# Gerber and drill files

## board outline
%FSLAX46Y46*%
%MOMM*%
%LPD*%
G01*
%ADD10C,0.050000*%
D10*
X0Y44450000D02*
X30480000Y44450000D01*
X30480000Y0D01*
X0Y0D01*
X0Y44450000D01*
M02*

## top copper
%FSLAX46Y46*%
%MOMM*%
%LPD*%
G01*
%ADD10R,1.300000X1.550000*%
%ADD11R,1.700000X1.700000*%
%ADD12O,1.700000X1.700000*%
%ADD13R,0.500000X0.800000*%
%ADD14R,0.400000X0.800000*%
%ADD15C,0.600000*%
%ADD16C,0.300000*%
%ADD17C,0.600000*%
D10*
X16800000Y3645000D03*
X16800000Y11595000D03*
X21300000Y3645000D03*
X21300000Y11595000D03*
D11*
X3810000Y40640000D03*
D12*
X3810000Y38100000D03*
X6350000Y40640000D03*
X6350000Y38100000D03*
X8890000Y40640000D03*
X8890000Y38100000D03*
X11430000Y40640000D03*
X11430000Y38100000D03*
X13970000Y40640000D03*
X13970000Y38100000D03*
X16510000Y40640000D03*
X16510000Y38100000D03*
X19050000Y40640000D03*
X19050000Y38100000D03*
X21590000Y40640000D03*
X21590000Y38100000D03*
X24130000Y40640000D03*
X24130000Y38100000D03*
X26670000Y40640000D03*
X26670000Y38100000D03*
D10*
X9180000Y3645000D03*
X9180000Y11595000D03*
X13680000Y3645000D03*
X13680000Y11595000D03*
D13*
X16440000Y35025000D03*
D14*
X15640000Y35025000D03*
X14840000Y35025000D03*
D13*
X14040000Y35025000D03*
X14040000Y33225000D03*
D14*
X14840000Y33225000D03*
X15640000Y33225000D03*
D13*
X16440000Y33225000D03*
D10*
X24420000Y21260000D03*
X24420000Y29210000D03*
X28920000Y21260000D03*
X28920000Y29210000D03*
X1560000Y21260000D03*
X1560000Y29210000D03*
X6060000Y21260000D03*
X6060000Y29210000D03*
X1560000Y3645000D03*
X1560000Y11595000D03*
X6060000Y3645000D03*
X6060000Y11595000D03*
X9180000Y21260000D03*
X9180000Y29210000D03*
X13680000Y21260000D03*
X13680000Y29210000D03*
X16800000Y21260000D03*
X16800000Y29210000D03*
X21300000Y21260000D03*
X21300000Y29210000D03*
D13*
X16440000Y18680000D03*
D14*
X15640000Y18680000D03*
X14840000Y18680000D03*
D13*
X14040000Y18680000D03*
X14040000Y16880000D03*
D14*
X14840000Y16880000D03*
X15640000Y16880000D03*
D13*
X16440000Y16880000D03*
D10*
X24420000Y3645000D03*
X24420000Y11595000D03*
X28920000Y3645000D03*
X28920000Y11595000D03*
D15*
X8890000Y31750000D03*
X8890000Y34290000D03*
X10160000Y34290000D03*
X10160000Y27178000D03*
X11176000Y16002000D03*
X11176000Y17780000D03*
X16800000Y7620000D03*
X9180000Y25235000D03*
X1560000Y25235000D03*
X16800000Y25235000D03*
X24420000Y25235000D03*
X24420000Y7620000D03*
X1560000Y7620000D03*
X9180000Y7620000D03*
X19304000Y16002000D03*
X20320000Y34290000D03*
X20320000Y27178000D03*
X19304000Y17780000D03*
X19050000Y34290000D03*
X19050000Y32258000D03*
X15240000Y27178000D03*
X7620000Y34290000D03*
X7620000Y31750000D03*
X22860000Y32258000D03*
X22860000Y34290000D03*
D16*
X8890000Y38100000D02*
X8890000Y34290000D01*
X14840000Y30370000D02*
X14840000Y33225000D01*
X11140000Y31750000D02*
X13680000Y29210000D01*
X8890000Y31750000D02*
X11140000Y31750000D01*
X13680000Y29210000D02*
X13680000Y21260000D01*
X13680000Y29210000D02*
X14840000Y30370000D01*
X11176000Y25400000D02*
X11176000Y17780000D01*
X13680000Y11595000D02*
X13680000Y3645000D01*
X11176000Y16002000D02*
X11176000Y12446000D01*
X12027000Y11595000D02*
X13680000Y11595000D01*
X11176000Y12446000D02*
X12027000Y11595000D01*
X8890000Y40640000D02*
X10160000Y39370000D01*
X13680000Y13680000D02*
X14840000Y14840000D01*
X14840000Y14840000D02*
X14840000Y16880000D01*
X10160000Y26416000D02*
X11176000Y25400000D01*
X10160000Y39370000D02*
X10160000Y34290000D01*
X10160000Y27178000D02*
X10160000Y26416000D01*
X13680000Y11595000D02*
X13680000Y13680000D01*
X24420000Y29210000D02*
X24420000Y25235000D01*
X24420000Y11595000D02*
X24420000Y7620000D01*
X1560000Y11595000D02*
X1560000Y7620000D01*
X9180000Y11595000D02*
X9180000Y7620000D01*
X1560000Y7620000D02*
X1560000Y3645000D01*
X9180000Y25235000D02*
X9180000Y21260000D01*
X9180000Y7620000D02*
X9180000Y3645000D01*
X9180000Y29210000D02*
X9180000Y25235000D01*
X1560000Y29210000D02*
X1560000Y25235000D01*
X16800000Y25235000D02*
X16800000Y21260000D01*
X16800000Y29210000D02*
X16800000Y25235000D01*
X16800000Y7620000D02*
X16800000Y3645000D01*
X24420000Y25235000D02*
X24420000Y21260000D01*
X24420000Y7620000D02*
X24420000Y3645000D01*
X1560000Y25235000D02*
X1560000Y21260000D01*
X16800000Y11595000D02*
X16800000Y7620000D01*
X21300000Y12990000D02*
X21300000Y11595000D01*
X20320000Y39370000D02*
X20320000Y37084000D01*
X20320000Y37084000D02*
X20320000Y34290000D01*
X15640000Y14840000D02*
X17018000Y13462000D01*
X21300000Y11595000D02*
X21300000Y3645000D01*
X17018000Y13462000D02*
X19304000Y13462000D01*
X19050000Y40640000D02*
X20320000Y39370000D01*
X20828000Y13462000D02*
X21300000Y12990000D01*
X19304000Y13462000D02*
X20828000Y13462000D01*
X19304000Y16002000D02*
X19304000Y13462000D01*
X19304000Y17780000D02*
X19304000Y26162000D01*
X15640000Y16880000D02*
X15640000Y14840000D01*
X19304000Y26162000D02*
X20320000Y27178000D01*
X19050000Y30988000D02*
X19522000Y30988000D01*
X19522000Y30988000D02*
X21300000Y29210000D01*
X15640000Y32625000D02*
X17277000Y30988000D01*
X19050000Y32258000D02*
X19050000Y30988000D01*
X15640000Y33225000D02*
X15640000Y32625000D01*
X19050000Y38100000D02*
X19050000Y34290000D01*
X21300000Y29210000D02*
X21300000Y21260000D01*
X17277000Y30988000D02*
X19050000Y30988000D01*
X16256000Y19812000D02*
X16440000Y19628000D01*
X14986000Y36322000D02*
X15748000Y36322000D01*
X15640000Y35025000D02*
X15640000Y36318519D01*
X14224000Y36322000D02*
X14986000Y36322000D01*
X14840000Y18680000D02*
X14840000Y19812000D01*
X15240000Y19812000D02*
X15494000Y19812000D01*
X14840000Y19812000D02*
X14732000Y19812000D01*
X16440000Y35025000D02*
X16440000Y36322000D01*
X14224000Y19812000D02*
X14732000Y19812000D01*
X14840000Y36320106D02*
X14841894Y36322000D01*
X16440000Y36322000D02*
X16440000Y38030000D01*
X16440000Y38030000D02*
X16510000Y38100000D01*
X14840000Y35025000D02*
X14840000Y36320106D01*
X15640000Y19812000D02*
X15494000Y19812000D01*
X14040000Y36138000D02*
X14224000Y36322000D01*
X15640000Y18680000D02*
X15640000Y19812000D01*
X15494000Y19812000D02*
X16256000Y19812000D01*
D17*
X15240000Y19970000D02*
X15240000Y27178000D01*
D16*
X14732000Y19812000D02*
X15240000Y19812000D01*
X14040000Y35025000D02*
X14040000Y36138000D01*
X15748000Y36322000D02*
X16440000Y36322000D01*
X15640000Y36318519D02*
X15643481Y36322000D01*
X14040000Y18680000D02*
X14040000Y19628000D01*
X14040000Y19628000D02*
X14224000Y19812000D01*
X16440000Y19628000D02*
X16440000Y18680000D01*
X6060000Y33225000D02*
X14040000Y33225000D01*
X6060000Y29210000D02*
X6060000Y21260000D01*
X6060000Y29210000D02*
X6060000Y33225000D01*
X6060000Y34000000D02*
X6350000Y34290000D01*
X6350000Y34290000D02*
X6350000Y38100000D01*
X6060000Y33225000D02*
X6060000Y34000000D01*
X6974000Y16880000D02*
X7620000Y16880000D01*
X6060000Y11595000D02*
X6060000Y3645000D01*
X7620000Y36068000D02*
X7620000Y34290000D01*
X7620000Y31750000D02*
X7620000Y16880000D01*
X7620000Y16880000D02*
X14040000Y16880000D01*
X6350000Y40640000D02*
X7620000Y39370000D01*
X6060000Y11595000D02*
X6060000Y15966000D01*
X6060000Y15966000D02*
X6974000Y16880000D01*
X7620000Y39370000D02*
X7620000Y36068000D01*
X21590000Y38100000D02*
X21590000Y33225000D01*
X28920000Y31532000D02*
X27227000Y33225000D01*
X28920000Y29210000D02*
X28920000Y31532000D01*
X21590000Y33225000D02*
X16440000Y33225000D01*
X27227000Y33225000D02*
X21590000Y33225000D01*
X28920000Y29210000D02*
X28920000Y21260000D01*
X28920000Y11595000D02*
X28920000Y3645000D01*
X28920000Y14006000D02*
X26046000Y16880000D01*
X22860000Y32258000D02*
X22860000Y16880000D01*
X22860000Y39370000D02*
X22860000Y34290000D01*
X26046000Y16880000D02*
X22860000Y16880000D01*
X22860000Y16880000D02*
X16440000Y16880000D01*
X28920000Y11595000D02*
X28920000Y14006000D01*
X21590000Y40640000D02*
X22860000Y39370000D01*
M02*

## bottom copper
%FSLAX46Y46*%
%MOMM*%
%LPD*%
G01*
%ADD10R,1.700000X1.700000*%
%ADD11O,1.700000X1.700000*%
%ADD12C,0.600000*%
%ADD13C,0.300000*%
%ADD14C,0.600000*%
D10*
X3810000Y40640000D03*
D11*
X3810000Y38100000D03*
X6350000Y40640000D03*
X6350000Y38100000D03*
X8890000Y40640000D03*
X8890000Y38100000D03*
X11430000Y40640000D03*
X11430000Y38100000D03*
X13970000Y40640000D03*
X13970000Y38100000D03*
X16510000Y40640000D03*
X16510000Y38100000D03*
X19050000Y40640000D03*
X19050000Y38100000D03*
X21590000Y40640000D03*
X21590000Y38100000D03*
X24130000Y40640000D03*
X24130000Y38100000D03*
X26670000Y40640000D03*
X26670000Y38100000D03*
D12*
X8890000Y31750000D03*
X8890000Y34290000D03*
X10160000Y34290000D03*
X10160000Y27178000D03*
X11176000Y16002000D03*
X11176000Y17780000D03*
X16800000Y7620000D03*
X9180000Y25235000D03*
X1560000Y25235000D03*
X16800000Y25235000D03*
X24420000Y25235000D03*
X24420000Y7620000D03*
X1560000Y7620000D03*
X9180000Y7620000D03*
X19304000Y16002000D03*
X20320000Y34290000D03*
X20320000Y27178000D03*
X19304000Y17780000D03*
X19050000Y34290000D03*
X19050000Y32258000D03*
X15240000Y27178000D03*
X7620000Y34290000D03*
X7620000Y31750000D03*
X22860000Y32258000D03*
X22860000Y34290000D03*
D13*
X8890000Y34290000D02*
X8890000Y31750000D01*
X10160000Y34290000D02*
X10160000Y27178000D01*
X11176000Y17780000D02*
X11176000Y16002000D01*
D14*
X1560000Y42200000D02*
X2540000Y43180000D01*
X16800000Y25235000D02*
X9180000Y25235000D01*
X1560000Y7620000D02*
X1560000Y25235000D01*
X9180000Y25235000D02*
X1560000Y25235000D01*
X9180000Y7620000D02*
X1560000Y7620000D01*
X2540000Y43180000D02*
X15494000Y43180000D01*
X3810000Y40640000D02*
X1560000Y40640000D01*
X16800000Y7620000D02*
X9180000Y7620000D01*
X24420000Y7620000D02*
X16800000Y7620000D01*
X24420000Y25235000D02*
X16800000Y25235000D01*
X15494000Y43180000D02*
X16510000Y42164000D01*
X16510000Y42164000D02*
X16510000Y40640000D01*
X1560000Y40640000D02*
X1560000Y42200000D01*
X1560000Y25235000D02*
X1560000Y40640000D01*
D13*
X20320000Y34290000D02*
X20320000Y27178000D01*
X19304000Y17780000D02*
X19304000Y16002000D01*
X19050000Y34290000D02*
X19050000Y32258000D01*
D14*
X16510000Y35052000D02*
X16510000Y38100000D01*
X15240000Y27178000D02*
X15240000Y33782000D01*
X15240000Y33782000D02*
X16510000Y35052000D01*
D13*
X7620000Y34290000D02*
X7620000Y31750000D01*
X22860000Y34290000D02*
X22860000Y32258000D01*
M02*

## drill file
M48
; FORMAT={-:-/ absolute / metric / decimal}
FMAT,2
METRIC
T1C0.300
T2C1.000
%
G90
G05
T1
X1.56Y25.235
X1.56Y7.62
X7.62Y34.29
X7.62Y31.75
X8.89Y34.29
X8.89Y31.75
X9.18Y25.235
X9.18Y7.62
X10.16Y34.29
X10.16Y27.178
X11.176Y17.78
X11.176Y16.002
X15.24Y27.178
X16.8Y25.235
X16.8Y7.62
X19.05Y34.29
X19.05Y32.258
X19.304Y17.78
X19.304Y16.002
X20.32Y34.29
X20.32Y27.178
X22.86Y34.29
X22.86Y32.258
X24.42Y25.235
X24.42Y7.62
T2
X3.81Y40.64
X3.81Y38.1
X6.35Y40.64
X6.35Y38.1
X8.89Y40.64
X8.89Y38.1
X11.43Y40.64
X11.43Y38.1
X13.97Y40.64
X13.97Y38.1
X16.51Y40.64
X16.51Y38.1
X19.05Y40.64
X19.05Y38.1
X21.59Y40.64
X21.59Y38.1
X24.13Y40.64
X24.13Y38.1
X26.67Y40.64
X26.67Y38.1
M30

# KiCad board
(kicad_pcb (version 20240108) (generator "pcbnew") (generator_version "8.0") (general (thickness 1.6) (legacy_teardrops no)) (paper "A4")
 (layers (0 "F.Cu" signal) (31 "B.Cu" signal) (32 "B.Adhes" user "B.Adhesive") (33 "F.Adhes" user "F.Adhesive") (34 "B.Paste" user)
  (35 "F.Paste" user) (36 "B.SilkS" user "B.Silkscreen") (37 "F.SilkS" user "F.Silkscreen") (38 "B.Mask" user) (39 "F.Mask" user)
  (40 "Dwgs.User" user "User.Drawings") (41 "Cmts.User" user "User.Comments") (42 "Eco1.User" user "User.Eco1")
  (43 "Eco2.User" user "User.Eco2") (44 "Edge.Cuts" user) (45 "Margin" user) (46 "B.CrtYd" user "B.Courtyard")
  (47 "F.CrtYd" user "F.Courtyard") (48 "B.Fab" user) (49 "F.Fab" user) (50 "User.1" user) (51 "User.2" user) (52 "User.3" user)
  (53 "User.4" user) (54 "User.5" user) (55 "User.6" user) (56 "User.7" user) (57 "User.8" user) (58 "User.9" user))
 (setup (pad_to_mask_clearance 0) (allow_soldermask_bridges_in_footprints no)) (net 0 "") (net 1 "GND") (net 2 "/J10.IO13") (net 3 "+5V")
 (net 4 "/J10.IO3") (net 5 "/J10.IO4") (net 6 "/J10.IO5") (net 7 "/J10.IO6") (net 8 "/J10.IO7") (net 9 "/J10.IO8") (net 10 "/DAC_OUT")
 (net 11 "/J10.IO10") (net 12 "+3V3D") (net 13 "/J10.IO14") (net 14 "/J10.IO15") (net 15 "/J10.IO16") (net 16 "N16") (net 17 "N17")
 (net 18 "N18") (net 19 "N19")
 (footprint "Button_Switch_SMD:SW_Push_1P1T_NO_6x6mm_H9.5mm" (layer "F.Cu") (at 19.05 -7.62 90)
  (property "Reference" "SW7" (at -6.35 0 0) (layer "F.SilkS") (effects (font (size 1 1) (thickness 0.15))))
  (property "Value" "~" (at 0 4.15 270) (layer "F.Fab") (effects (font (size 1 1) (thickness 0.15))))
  (pad "1" smd rect (at -3.975 -2.25 90) (size 1.55 1.3) (layers "F.Cu" "F.Paste" "F.Mask") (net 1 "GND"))
  (pad "1" smd rect (at 3.975 -2.25 90) (size 1.55 1.3) (layers "F.Cu" "F.Paste" "F.Mask") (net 1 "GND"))
  (pad "2" smd rect (at -3.975 2.25 90) (size 1.55 1.3) (layers "F.Cu" "F.Paste" "F.Mask") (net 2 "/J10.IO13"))
  (pad "2" smd rect (at 3.975 2.25 90) (size 1.55 1.3) (layers "F.Cu" "F.Paste" "F.Mask") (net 2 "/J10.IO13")))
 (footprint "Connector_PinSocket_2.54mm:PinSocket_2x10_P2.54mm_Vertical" (layer "F.Cu") (at 3.81 -40.64 90)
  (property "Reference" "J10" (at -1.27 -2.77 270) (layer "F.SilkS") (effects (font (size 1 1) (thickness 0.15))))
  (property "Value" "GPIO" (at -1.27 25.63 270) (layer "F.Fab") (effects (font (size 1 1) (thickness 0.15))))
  (pad "1" thru_hole rect (at 0 0 90) (size 1.7 1.7) (drill 1) (layers "*.Cu" "*.Mask") (remove_unused_layers no) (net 1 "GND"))
  (pad "2" thru_hole oval (at -2.54 0 90) (size 1.7 1.7) (drill 1) (layers "*.Cu" "*.Mask") (remove_unused_layers no) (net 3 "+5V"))
  (pad "3" thru_hole oval (at 0 2.54 90) (size 1.7 1.7) (drill 1) (layers "*.Cu" "*.Mask") (remove_unused_layers no) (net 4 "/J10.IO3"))
  (pad "4" thru_hole oval (at -2.54 2.54 90) (size 1.7 1.7) (drill 1) (layers "*.Cu" "*.Mask") (remove_unused_layers no) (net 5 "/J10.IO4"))
  (pad "5" thru_hole oval (at 0 5.08 90) (size 1.7 1.7) (drill 1) (layers "*.Cu" "*.Mask") (remove_unused_layers no) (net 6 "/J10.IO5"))
  (pad "6" thru_hole oval (at -2.54 5.08 90) (size 1.7 1.7) (drill 1) (layers "*.Cu" "*.Mask") (remove_unused_layers no) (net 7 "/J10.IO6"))
  (pad "7" thru_hole oval (at 0 7.62 90) (size 1.7 1.7) (drill 1) (layers "*.Cu" "*.Mask") (remove_unused_layers no) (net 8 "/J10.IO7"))
  (pad "8" thru_hole oval (at -2.54 7.62 90) (size 1.7 1.7) (drill 1) (layers "*.Cu" "*.Mask") (remove_unused_layers no) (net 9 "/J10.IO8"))
  (pad "9" thru_hole oval (at 0 10.16 90) (size 1.7 1.7) (drill 1) (layers "*.Cu" "*.Mask") (remove_unused_layers no) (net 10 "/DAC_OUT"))
  (pad "10" thru_hole oval (at -2.54 10.16 90) (size 1.7 1.7) (drill 1) (layers "*.Cu" "*.Mask") (remove_unused_layers no)
   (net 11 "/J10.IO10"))
  (pad "11" thru_hole oval (at 0 12.7 90) (size 1.7 1.7) (drill 1) (layers "*.Cu" "*.Mask") (remove_unused_layers no) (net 1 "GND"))
  (pad "12" thru_hole oval (at -2.54 12.7 90) (size 1.7 1.7) (drill 1) (layers "*.Cu" "*.Mask") (remove_unused_layers no) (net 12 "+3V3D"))
  (pad "13" thru_hole oval (at 0 15.24 90) (size 1.7 1.7) (drill 1) (layers "*.Cu" "*.Mask") (remove_unused_layers no) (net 2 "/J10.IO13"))
  (pad "14" thru_hole oval (at -2.54 15.24 90) (size 1.7 1.7) (drill 1) (layers "*.Cu" "*.Mask") (remove_unused_layers no)
   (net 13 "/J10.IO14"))
  (pad "15" thru_hole oval (at 0 17.78 90) (size 1.7 1.7) (drill 1) (layers "*.Cu" "*.Mask") (remove_unused_layers no) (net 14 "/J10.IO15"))
  (pad "16" thru_hole oval (at -2.54 17.78 90) (size 1.7 1.7) (drill 1) (layers "*.Cu" "*.Mask") (remove_unused_layers no)
   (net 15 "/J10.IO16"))
  (pad "17" thru_hole oval (at 0 20.32 90) (size 1.7 1.7) (drill 1) (layers "*.Cu" "*.Mask") (remove_unused_layers no) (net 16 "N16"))
  (pad "18" thru_hole oval (at -2.54 20.32 90) (size 1.7 1.7) (drill 1) (layers "*.Cu" "*.Mask") (remove_unused_layers no) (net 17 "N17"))
  (pad "19" thru_hole oval (at 0 22.86 90) (size 1.7 1.7) (drill 1) (layers "*.Cu" "*.Mask") (remove_unused_layers no) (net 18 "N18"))
  (pad "20" thru_hole oval (at -2.54 22.86 90) (size 1.7 1.7) (drill 1) (layers "*.Cu" "*.Mask") (remove_unused_layers no) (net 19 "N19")))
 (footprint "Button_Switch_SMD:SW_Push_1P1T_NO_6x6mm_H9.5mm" (layer "F.Cu") (at 11.43 -7.62 90)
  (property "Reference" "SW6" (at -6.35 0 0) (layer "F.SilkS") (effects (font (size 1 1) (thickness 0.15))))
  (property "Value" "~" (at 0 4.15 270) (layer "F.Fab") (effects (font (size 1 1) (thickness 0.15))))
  (pad "1" smd rect (at -3.975 -2.25 90) (size 1.55 1.3) (layers "F.Cu" "F.Paste" "F.Mask") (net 1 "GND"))
  (pad "1" smd rect (at 3.975 -2.25 90) (size 1.55 1.3) (layers "F.Cu" "F.Paste" "F.Mask") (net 1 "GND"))
  (pad "2" smd rect (at -3.975 2.25 90) (size 1.55 1.3) (layers "F.Cu" "F.Paste" "F.Mask") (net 6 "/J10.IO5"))
  (pad "2" smd rect (at 3.975 2.25 90) (size 1.55 1.3) (layers "F.Cu" "F.Paste" "F.Mask") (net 6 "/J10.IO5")))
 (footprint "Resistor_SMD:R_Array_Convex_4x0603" (layer "F.Cu") (at 15.24 -34.125 -90)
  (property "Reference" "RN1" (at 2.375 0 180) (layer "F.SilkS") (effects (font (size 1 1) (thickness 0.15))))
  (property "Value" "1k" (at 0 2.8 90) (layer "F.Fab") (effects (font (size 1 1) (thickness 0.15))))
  (pad "1" smd rect (at -0.9 -1.2 270) (size 0.8 0.5) (layers "F.Cu" "F.Paste" "F.Mask") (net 12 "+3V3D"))
  (pad "2" smd rect (at -0.9 -0.4 270) (size 0.8 0.4) (layers "F.Cu" "F.Paste" "F.Mask") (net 12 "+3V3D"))
  (pad "3" smd rect (at -0.9 0.4 270) (size 0.8 0.4) (layers "F.Cu" "F.Paste" "F.Mask") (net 12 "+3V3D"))
  (pad "4" smd rect (at -0.9 1.2 270) (size 0.8 0.5) (layers "F.Cu" "F.Paste" "F.Mask") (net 12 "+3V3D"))
  (pad "5" smd rect (at 0.9 1.2 270) (size 0.8 0.5) (layers "F.Cu" "F.Paste" "F.Mask") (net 5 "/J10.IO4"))
  (pad "6" smd rect (at 0.9 0.4 270) (size 0.8 0.4) (layers "F.Cu" "F.Paste" "F.Mask") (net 7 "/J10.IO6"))
  (pad "7" smd rect (at 0.9 -0.4 270) (size 0.8 0.4) (layers "F.Cu" "F.Paste" "F.Mask") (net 13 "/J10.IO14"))
  (pad "8" smd rect (at 0.9 -1.2 270) (size 0.8 0.5) (layers "F.Cu" "F.Paste" "F.Mask") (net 15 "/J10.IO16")))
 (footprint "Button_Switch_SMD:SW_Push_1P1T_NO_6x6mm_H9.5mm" (layer "F.Cu") (at 26.67 -25.235 90)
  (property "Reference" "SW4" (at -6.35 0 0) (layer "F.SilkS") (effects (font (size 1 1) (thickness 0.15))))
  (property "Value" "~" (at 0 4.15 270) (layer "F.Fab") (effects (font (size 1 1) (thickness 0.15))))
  (pad "1" smd rect (at -3.975 -2.25 90) (size 1.55 1.3) (layers "F.Cu" "F.Paste" "F.Mask") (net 1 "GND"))
  (pad "1" smd rect (at 3.975 -2.25 90) (size 1.55 1.3) (layers "F.Cu" "F.Paste" "F.Mask") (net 1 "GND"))
  (pad "2" smd rect (at -3.975 2.25 90) (size 1.55 1.3) (layers "F.Cu" "F.Paste" "F.Mask") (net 15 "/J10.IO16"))
  (pad "2" smd rect (at 3.975 2.25 90) (size 1.55 1.3) (layers "F.Cu" "F.Paste" "F.Mask") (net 15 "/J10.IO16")))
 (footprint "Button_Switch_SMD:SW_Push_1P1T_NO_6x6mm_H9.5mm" (layer "F.Cu") (at 3.81 -25.235 90)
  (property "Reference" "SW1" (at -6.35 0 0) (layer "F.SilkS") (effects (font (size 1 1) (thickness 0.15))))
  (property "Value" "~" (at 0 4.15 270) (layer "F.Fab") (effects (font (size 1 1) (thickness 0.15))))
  (pad "1" smd rect (at -3.975 -2.25 90) (size 1.55 1.3) (layers "F.Cu" "F.Paste" "F.Mask") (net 1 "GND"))
  (pad "1" smd rect (at 3.975 -2.25 90) (size 1.55 1.3) (layers "F.Cu" "F.Paste" "F.Mask") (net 1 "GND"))
  (pad "2" smd rect (at -3.975 2.25 90) (size 1.55 1.3) (layers "F.Cu" "F.Paste" "F.Mask") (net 5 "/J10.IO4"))
  (pad "2" smd rect (at 3.975 2.25 90) (size 1.55 1.3) (layers "F.Cu" "F.Paste" "F.Mask") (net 5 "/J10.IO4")))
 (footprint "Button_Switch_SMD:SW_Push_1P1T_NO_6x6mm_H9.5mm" (layer "F.Cu") (at 3.81 -7.62 90)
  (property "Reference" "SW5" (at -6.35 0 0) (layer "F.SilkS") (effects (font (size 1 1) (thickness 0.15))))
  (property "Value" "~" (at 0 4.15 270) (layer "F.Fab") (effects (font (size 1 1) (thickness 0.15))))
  (pad "1" smd rect (at -3.975 -2.25 90) (size 1.55 1.3) (layers "F.Cu" "F.Paste" "F.Mask") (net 1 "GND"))
  (pad "1" smd rect (at 3.975 -2.25 90) (size 1.55 1.3) (layers "F.Cu" "F.Paste" "F.Mask") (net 1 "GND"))
  (pad "2" smd rect (at -3.975 2.25 90) (size 1.55 1.3) (layers "F.Cu" "F.Paste" "F.Mask") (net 4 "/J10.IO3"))
  (pad "2" smd rect (at 3.975 2.25 90) (size 1.55 1.3) (layers "F.Cu" "F.Paste" "F.Mask") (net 4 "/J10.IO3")))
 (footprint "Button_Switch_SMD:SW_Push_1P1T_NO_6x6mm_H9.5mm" (layer "F.Cu") (at 11.43 -25.235 90)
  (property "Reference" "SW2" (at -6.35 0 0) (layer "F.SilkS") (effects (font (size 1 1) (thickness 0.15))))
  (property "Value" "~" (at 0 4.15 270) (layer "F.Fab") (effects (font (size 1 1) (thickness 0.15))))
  (pad "1" smd rect (at -3.975 -2.25 90) (size 1.55 1.3) (layers "F.Cu" "F.Paste" "F.Mask") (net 1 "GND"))
  (pad "1" smd rect (at 3.975 -2.25 90) (size 1.55 1.3) (layers "F.Cu" "F.Paste" "F.Mask") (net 1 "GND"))
  (pad "2" smd rect (at -3.975 2.25 90) (size 1.55 1.3) (layers "F.Cu" "F.Paste" "F.Mask") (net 7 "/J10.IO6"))
  (pad "2" smd rect (at 3.975 2.25 90) (size 1.55 1.3) (layers "F.Cu" "F.Paste" "F.Mask") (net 7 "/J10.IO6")))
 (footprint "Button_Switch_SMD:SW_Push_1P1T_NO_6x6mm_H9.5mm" (layer "F.Cu") (at 19.05 -25.235 90)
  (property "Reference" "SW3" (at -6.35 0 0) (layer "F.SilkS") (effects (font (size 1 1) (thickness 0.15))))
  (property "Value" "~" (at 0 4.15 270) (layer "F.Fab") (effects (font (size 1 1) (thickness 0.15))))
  (pad "1" smd rect (at -3.975 -2.25 90) (size 1.55 1.3) (layers "F.Cu" "F.Paste" "F.Mask") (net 1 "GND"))
  (pad "1" smd rect (at 3.975 -2.25 90) (size 1.55 1.3) (layers "F.Cu" "F.Paste" "F.Mask") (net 1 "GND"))
  (pad "2" smd rect (at -3.975 2.25 90) (size 1.55 1.3) (layers "F.Cu" "F.Paste" "F.Mask") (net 13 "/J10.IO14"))
  (pad "2" smd rect (at 3.975 2.25 90) (size 1.55 1.3) (layers "F.Cu" "F.Paste" "F.Mask") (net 13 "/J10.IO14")))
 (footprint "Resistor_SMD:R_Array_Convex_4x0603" (layer "F.Cu") (at 15.24 -17.78 -90)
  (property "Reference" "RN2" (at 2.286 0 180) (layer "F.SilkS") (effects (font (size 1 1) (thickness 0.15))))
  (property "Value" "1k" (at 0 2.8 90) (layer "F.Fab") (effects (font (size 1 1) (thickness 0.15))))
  (pad "1" smd rect (at -0.9 -1.2 270) (size 0.8 0.5) (layers "F.Cu" "F.Paste" "F.Mask") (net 12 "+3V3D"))
  (pad "2" smd rect (at -0.9 -0.4 270) (size 0.8 0.4) (layers "F.Cu" "F.Paste" "F.Mask") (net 12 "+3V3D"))
  (pad "3" smd rect (at -0.9 0.4 270) (size 0.8 0.4) (layers "F.Cu" "F.Paste" "F.Mask") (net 12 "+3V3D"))
  (pad "4" smd rect (at -0.9 1.2 270) (size 0.8 0.5) (layers "F.Cu" "F.Paste" "F.Mask") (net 12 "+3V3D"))
  (pad "5" smd rect (at 0.9 1.2 270) (size 0.8 0.5) (layers "F.Cu" "F.Paste" "F.Mask") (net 4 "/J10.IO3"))
  (pad "6" smd rect (at 0.9 0.4 270) (size 0.8 0.4) (layers "F.Cu" "F.Paste" "F.Mask") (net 6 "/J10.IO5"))
  (pad "7" smd rect (at 0.9 -0.4 270) (size 0.8 0.4) (layers "F.Cu" "F.Paste" "F.Mask") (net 2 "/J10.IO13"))
  (pad "8" smd rect (at 0.9 -1.2 270) (size 0.8 0.5) (layers "F.Cu" "F.Paste" "F.Mask") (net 14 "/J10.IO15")))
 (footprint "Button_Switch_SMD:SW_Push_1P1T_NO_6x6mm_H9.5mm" (layer "F.Cu") (at 26.67 -7.62 90)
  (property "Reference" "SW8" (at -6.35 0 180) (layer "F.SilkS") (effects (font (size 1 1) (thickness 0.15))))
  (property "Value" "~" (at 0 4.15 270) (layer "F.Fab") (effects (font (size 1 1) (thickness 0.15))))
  (pad "1" smd rect (at -3.975 -2.25 90) (size 1.55 1.3) (layers "F.Cu" "F.Paste" "F.Mask") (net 1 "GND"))
  (pad "1" smd rect (at 3.975 -2.25 90) (size 1.55 1.3) (layers "F.Cu" "F.Paste" "F.Mask") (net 1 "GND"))
  (pad "2" smd rect (at -3.975 2.25 90) (size 1.55 1.3) (layers "F.Cu" "F.Paste" "F.Mask") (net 14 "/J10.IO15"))
  (pad "2" smd rect (at 3.975 2.25 90) (size 1.55 1.3) (layers "F.Cu" "F.Paste" "F.Mask") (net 14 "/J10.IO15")))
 (gr_rect (start 0 -44.45) (end 30.48 0) (stroke (width 0.05) (type default)) (fill none) (layer "Edge.Cuts"))
 (segment (start 8.89 -38.1) (end 8.89 -34.29) (width 0.3) (layer "F.Cu") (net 7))
 (segment (start 14.84 -30.37) (end 14.84 -33.225) (width 0.3) (layer "F.Cu") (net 7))
 (segment (start 11.14 -31.75) (end 13.68 -29.21) (width 0.3) (layer "F.Cu") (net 7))
 (segment (start 8.89 -31.75) (end 11.14 -31.75) (width 0.3) (layer "F.Cu") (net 7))
 (segment (start 13.68 -29.21) (end 13.68 -21.26) (width 0.3) (layer "F.Cu") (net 7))
 (segment (start 13.68 -29.21) (end 14.84 -30.37) (width 0.3) (layer "F.Cu") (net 7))
 (via (at 8.89 -31.75) (size 0.6) (drill 0.3) (layers "F.Cu" "B.Cu") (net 7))
 (via (at 8.89 -34.29) (size 0.6) (drill 0.3) (layers "F.Cu" "B.Cu") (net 7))
 (segment (start 8.89 -34.29) (end 8.89 -31.75) (width 0.3) (layer "B.Cu") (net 7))
 (segment (start 11.176 -25.4) (end 11.176 -17.78) (width 0.3) (layer "F.Cu") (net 6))
 (segment (start 13.68 -11.595) (end 13.68 -3.645) (width 0.3) (layer "F.Cu") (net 6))
 (segment (start 11.176 -16.002) (end 11.176 -12.446) (width 0.3) (layer "F.Cu") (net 6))
 (segment (start 12.027 -11.595) (end 13.68 -11.595) (width 0.3) (layer "F.Cu") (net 6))
 (segment (start 11.176 -12.446) (end 12.027 -11.595) (width 0.3) (layer "F.Cu") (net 6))
 (segment (start 8.89 -40.64) (end 10.16 -39.37) (width 0.3) (layer "F.Cu") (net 6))
 (segment (start 13.68 -13.68) (end 14.84 -14.84) (width 0.3) (layer "F.Cu") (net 6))
 (segment (start 14.84 -14.84) (end 14.84 -16.88) (width 0.3) (layer "F.Cu") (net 6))
 (segment (start 10.16 -26.416) (end 11.176 -25.4) (width 0.3) (layer "F.Cu") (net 6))
 (segment (start 10.16 -39.37) (end 10.16 -34.29) (width 0.3) (layer "F.Cu") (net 6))
 (segment (start 10.16 -27.178) (end 10.16 -26.416) (width 0.3) (layer "F.Cu") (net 6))
 (segment (start 13.68 -11.595) (end 13.68 -13.68) (width 0.3) (layer "F.Cu") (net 6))
 (via (at 10.16 -34.29) (size 0.6) (drill 0.3) (layers "F.Cu" "B.Cu") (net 6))
 (via (at 10.16 -27.178) (size 0.6) (drill 0.3) (layers "F.Cu" "B.Cu") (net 6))
 (via (at 11.176 -16.002) (size 0.6) (drill 0.3) (layers "F.Cu" "B.Cu") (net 6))
 (via (at 11.176 -17.78) (size 0.6) (drill 0.3) (layers "F.Cu" "B.Cu") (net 6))
 (segment (start 10.16 -34.29) (end 10.16 -27.178) (width 0.3) (layer "B.Cu") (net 6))
 (segment (start 11.176 -17.78) (end 11.176 -16.002) (width 0.3) (layer "B.Cu") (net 6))
 (segment (start 24.42 -29.21) (end 24.42 -25.235) (width 0.3) (layer "F.Cu") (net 1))
 (segment (start 24.42 -11.595) (end 24.42 -7.62) (width 0.3) (layer "F.Cu") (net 1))
 (segment (start 1.56 -11.595) (end 1.56 -7.62) (width 0.3) (layer "F.Cu") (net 1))
 (segment (start 9.18 -11.595) (end 9.18 -7.62) (width 0.3) (layer "F.Cu") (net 1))
 (segment (start 1.56 -7.62) (end 1.56 -3.645) (width 0.3) (layer "F.Cu") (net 1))
 (segment (start 9.18 -25.235) (end 9.18 -21.26) (width 0.3) (layer "F.Cu") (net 1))
 (segment (start 9.18 -7.62) (end 9.18 -3.645) (width 0.3) (layer "F.Cu") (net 1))
 (segment (start 9.18 -29.21) (end 9.18 -25.235) (width 0.3) (layer "F.Cu") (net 1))
 (segment (start 1.56 -29.21) (end 1.56 -25.235) (width 0.3) (layer "F.Cu") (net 1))
 (segment (start 16.8 -25.235) (end 16.8 -21.26) (width 0.3) (layer "F.Cu") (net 1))
 (segment (start 16.8 -29.21) (end 16.8 -25.235) (width 0.3) (layer "F.Cu") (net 1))
 (segment (start 16.8 -7.62) (end 16.8 -3.645) (width 0.3) (layer "F.Cu") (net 1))
 (segment (start 24.42 -25.235) (end 24.42 -21.26) (width 0.3) (layer "F.Cu") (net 1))
 (segment (start 24.42 -7.62) (end 24.42 -3.645) (width 0.3) (layer "F.Cu") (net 1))
 (segment (start 1.56 -25.235) (end 1.56 -21.26) (width 0.3) (layer "F.Cu") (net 1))
 (segment (start 16.8 -11.595) (end 16.8 -7.62) (width 0.3) (layer "F.Cu") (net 1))
 (via (at 16.8 -7.62) (size 0.6) (drill 0.3) (layers "F.Cu" "B.Cu") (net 1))
 (via (at 9.18 -25.235) (size 0.6) (drill 0.3) (layers "F.Cu" "B.Cu") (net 1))
 (via (at 1.56 -25.235) (size 0.6) (drill 0.3) (layers "F.Cu" "B.Cu") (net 1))
 (via (at 16.8 -25.235) (size 0.6) (drill 0.3) (layers "F.Cu" "B.Cu") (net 1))
 (via (at 24.42 -25.235) (size 0.6) (drill 0.3) (layers "F.Cu" "B.Cu") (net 1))
 (via (at 24.42 -7.62) (size 0.6) (drill 0.3) (layers "F.Cu" "B.Cu") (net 1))
 (via (at 1.56 -7.62) (size 0.6) (drill 0.3) (layers "F.Cu" "B.Cu") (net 1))
 (via (at 9.18 -7.62) (size 0.6) (drill 0.3) (layers "F.Cu" "B.Cu") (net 1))
 (segment (start 1.56 -42.2) (end 2.54 -43.18) (width 0.6) (layer "B.Cu") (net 1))
 (segment (start 16.8 -25.235) (end 9.18 -25.235) (width 0.6) (layer "B.Cu") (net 1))
 (segment (start 1.56 -7.62) (end 1.56 -25.235) (width 0.6) (layer "B.Cu") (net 1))
 (segment (start 9.18 -25.235) (end 1.56 -25.235) (width 0.6) (layer "B.Cu") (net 1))
 (segment (start 9.18 -7.62) (end 1.56 -7.62) (width 0.6) (layer "B.Cu") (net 1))
 (segment (start 2.54 -43.18) (end 15.494 -43.18) (width 0.6) (layer "B.Cu") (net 1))
 (segment (start 3.81 -40.64) (end 1.56 -40.64) (width 0.6) (layer "B.Cu") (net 1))
 (segment (start 16.8 -7.62) (end 9.18 -7.62) (width 0.6) (layer "B.Cu") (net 1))
 (segment (start 24.42 -7.62) (end 16.8 -7.62) (width 0.6) (layer "B.Cu") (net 1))
 (segment (start 24.42 -25.235) (end 16.8 -25.235) (width 0.6) (layer "B.Cu") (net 1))
 (segment (start 15.494 -43.18) (end 16.51 -42.164) (width 0.6) (layer "B.Cu") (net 1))
 (segment (start 16.51 -42.164) (end 16.51 -40.64) (width 0.6) (layer "B.Cu") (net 1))
 (segment (start 1.56 -40.64) (end 1.56 -42.2) (width 0.6) (layer "B.Cu") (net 1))
 (segment (start 1.56 -25.235) (end 1.56 -40.64) (width 0.6) (layer "B.Cu") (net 1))
 (segment (start 21.3 -12.99) (end 21.3 -11.595) (width 0.3) (layer "F.Cu") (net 2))
 (segment (start 20.32 -39.37) (end 20.32 -37.084) (width 0.3) (layer "F.Cu") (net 2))
 (segment (start 20.32 -37.084) (end 20.32 -34.29) (width 0.3) (layer "F.Cu") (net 2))
 (segment (start 15.64 -14.84) (end 17.018 -13.462) (width 0.3) (layer "F.Cu") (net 2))
 (segment (start 21.3 -11.595) (end 21.3 -3.645) (width 0.3) (layer "F.Cu") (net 2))
 (segment (start 17.018 -13.462) (end 19.304 -13.462) (width 0.3) (layer "F.Cu") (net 2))
 (segment (start 19.05 -40.64) (end 20.32 -39.37) (width 0.3) (layer "F.Cu") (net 2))
 (segment (start 20.828 -13.462) (end 21.3 -12.99) (width 0.3) (layer "F.Cu") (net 2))
 (segment (start 19.304 -13.462) (end 20.828 -13.462) (width 0.3) (layer "F.Cu") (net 2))
 (segment (start 19.304 -16.002) (end 19.304 -13.462) (width 0.3) (layer "F.Cu") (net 2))
 (segment (start 19.304 -17.78) (end 19.304 -26.162) (width 0.3) (layer "F.Cu") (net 2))
 (segment (start 15.64 -16.88) (end 15.64 -14.84) (width 0.3) (layer "F.Cu") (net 2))
 (segment (start 19.304 -26.162) (end 20.32 -27.178) (width 0.3) (layer "F.Cu") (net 2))
 (via (at 19.304 -16.002) (size 0.6) (drill 0.3) (layers "F.Cu" "B.Cu") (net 2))
 (via (at 20.32 -34.29) (size 0.6) (drill 0.3) (layers "F.Cu" "B.Cu") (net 2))
 (via (at 20.32 -27.178) (size 0.6) (drill 0.3) (layers "F.Cu" "B.Cu") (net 2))
 (via (at 19.304 -17.78) (size 0.6) (drill 0.3) (layers "F.Cu" "B.Cu") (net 2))
 (segment (start 20.32 -34.29) (end 20.32 -27.178) (width 0.3) (layer "B.Cu") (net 2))
 (segment (start 19.304 -17.78) (end 19.304 -16.002) (width 0.3) (layer "B.Cu") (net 2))
 (segment (start 19.05 -30.988) (end 19.522 -30.988) (width 0.3) (layer "F.Cu") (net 13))
 (segment (start 19.522 -30.988) (end 21.3 -29.21) (width 0.3) (layer "F.Cu") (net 13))
 (segment (start 15.64 -32.625) (end 17.277 -30.988) (width 0.3) (layer "F.Cu") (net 13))
 (segment (start 19.05 -32.258) (end 19.05 -30.988) (width 0.3) (layer "F.Cu") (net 13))
 (segment (start 15.64 -33.225) (end 15.64 -32.625) (width 0.3) (layer "F.Cu") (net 13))
 (segment (start 19.05 -38.1) (end 19.05 -34.29) (width 0.3) (layer "F.Cu") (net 13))
 (segment (start 21.3 -29.21) (end 21.3 -21.26) (width 0.3) (layer "F.Cu") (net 13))
 (segment (start 17.277 -30.988) (end 19.05 -30.988) (width 0.3) (layer "F.Cu") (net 13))
 (via (at 19.05 -34.29) (size 0.6) (drill 0.3) (layers "F.Cu" "B.Cu") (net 13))
 (via (at 19.05 -32.258) (size 0.6) (drill 0.3) (layers "F.Cu" "B.Cu") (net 13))
 (segment (start 19.05 -34.29) (end 19.05 -32.258) (width 0.3) (layer "B.Cu") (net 13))
 (segment (start 16.256 -19.812) (end 16.44 -19.628) (width 0.3) (layer "F.Cu") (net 12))
 (segment (start 14.986 -36.322) (end 15.748 -36.322) (width 0.3) (layer "F.Cu") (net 12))
 (segment (start 15.64 -35.025) (end 15.64 -36.318519) (width 0.3) (layer "F.Cu") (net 12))
 (segment (start 14.224 -36.322) (end 14.986 -36.322) (width 0.3) (layer "F.Cu") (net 12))
 (segment (start 14.84 -18.68) (end 14.84 -19.812) (width 0.3) (layer "F.Cu") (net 12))
 (segment (start 15.24 -19.812) (end 15.494 -19.812) (width 0.3) (layer "F.Cu") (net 12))
 (segment (start 14.84 -19.812) (end 14.732 -19.812) (width 0.3) (layer "F.Cu") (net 12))
 (segment (start 16.44 -35.025) (end 16.44 -36.322) (width 0.3) (layer "F.Cu") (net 12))
 (segment (start 14.224 -19.812) (end 14.732 -19.812) (width 0.3) (layer "F.Cu") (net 12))
 (segment (start 14.84 -36.320106) (end 14.841894 -36.322) (width 0.3) (layer "F.Cu") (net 12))
 (segment (start 16.44 -36.322) (end 16.44 -38.03) (width 0.3) (layer "F.Cu") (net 12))
 (segment (start 16.44 -38.03) (end 16.51 -38.1) (width 0.3) (layer "F.Cu") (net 12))
 (segment (start 14.84 -35.025) (end 14.84 -36.320106) (width 0.3) (layer "F.Cu") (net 12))
 (segment (start 15.64 -19.812) (end 15.494 -19.812) (width 0.3) (layer "F.Cu") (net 12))
 (segment (start 14.04 -36.138) (end 14.224 -36.322) (width 0.3) (layer "F.Cu") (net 12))
 (segment (start 15.64 -18.68) (end 15.64 -19.812) (width 0.3) (layer "F.Cu") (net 12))
 (segment (start 15.494 -19.812) (end 16.256 -19.812) (width 0.3) (layer "F.Cu") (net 12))
 (segment (start 15.24 -19.97) (end 15.24 -27.178) (width 0.6) (layer "F.Cu") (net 12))
 (segment (start 14.732 -19.812) (end 15.24 -19.812) (width 0.3) (layer "F.Cu") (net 12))
 (segment (start 14.04 -35.025) (end 14.04 -36.138) (width 0.3) (layer "F.Cu") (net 12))
 (segment (start 15.748 -36.322) (end 16.44 -36.322) (width 0.3) (layer "F.Cu") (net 12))
 (segment (start 15.64 -36.318519) (end 15.643481 -36.322) (width 0.3) (layer "F.Cu") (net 12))
 (segment (start 14.04 -18.68) (end 14.04 -19.628) (width 0.3) (layer "F.Cu") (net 12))
 (segment (start 14.04 -19.628) (end 14.224 -19.812) (width 0.3) (layer "F.Cu") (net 12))
 (segment (start 16.44 -19.628) (end 16.44 -18.68) (width 0.3) (layer "F.Cu") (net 12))
 (via (at 15.24 -27.178) (size 0.6) (drill 0.3) (layers "F.Cu" "B.Cu") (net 12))
 (segment (start 16.51 -35.052) (end 16.51 -38.1) (width 0.6) (layer "B.Cu") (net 12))
 (segment (start 15.24 -27.178) (end 15.24 -33.782) (width 0.6) (layer "B.Cu") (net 12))
 (segment (start 15.24 -33.782) (end 16.51 -35.052) (width 0.6) (layer "B.Cu") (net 12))
 (segment (start 6.06 -33.225) (end 14.04 -33.225) (width 0.3) (layer "F.Cu") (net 5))
 (segment (start 6.06 -29.21) (end 6.06 -21.26) (width 0.3) (layer "F.Cu") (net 5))
 (segment (start 6.06 -29.21) (end 6.06 -33.225) (width 0.3) (layer "F.Cu") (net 5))
 (segment (start 6.06 -34) (end 6.35 -34.29) (width 0.3) (layer "F.Cu") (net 5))
 (segment (start 6.35 -34.29) (end 6.35 -38.1) (width 0.3) (layer "F.Cu") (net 5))
 (segment (start 6.06 -33.225) (end 6.06 -34) (width 0.3) (layer "F.Cu") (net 5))
 (segment (start 6.974 -16.88) (end 7.62 -16.88) (width 0.3) (layer "F.Cu") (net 4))
 (segment (start 6.06 -11.595) (end 6.06 -3.645) (width 0.3) (layer "F.Cu") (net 4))
 (segment (start 7.62 -36.068) (end 7.62 -34.29) (width 0.3) (layer "F.Cu") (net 4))
 (segment (start 7.62 -31.75) (end 7.62 -16.88) (width 0.3) (layer "F.Cu") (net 4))
 (segment (start 7.62 -16.88) (end 14.04 -16.88) (width 0.3) (layer "F.Cu") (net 4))
 (segment (start 6.35 -40.64) (end 7.62 -39.37) (width 0.3) (layer "F.Cu") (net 4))
 (segment (start 6.06 -11.595) (end 6.06 -15.966) (width 0.3) (layer "F.Cu") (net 4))
 (segment (start 6.06 -15.966) (end 6.974 -16.88) (width 0.3) (layer "F.Cu") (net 4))
 (segment (start 7.62 -39.37) (end 7.62 -36.068) (width 0.3) (layer "F.Cu") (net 4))
 (via (at 7.62 -34.29) (size 0.6) (drill 0.3) (layers "F.Cu" "B.Cu") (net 4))
 (via (at 7.62 -31.75) (size 0.6) (drill 0.3) (layers "F.Cu" "B.Cu") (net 4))
 (segment (start 7.62 -34.29) (end 7.62 -31.75) (width 0.3) (layer "B.Cu") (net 4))
 (segment (start 21.59 -38.1) (end 21.59 -33.225) (width 0.3) (layer "F.Cu") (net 15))
 (segment (start 28.92 -31.532) (end 27.227 -33.225) (width 0.3) (layer "F.Cu") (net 15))
 (segment (start 28.92 -29.21) (end 28.92 -31.532) (width 0.3) (layer "F.Cu") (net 15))
 (segment (start 21.59 -33.225) (end 16.44 -33.225) (width 0.3) (layer "F.Cu") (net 15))
 (segment (start 27.227 -33.225) (end 21.59 -33.225) (width 0.3) (layer "F.Cu") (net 15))
 (segment (start 28.92 -29.21) (end 28.92 -21.26) (width 0.3) (layer "F.Cu") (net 15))
 (segment (start 28.92 -11.595) (end 28.92 -3.645) (width 0.3) (layer "F.Cu") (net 14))
 (segment (start 28.92 -14.006) (end 26.046 -16.88) (width 0.3) (layer "F.Cu") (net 14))
 (segment (start 22.86 -32.258) (end 22.86 -16.88) (width 0.3) (layer "F.Cu") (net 14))
 (segment (start 22.86 -39.37) (end 22.86 -34.29) (width 0.3) (layer "F.Cu") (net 14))
 (segment (start 26.046 -16.88) (end 22.86 -16.88) (width 0.3) (layer "F.Cu") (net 14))
 (segment (start 22.86 -16.88) (end 16.44 -16.88) (width 0.3) (layer "F.Cu") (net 14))
 (segment (start 28.92 -11.595) (end 28.92 -14.006) (width 0.3) (layer "F.Cu") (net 14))
 (segment (start 21.59 -40.64) (end 22.86 -39.37) (width 0.3) (layer "F.Cu") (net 14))
 (via (at 22.86 -32.258) (size 0.6) (drill 0.3) (layers "F.Cu" "B.Cu") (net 14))
 (via (at 22.86 -34.29) (size 0.6) (drill 0.3) (layers "F.Cu" "B.Cu") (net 14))
 (segment (start 22.86 -34.29) (end 22.86 -32.258) (width 0.3) (layer "B.Cu") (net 14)))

